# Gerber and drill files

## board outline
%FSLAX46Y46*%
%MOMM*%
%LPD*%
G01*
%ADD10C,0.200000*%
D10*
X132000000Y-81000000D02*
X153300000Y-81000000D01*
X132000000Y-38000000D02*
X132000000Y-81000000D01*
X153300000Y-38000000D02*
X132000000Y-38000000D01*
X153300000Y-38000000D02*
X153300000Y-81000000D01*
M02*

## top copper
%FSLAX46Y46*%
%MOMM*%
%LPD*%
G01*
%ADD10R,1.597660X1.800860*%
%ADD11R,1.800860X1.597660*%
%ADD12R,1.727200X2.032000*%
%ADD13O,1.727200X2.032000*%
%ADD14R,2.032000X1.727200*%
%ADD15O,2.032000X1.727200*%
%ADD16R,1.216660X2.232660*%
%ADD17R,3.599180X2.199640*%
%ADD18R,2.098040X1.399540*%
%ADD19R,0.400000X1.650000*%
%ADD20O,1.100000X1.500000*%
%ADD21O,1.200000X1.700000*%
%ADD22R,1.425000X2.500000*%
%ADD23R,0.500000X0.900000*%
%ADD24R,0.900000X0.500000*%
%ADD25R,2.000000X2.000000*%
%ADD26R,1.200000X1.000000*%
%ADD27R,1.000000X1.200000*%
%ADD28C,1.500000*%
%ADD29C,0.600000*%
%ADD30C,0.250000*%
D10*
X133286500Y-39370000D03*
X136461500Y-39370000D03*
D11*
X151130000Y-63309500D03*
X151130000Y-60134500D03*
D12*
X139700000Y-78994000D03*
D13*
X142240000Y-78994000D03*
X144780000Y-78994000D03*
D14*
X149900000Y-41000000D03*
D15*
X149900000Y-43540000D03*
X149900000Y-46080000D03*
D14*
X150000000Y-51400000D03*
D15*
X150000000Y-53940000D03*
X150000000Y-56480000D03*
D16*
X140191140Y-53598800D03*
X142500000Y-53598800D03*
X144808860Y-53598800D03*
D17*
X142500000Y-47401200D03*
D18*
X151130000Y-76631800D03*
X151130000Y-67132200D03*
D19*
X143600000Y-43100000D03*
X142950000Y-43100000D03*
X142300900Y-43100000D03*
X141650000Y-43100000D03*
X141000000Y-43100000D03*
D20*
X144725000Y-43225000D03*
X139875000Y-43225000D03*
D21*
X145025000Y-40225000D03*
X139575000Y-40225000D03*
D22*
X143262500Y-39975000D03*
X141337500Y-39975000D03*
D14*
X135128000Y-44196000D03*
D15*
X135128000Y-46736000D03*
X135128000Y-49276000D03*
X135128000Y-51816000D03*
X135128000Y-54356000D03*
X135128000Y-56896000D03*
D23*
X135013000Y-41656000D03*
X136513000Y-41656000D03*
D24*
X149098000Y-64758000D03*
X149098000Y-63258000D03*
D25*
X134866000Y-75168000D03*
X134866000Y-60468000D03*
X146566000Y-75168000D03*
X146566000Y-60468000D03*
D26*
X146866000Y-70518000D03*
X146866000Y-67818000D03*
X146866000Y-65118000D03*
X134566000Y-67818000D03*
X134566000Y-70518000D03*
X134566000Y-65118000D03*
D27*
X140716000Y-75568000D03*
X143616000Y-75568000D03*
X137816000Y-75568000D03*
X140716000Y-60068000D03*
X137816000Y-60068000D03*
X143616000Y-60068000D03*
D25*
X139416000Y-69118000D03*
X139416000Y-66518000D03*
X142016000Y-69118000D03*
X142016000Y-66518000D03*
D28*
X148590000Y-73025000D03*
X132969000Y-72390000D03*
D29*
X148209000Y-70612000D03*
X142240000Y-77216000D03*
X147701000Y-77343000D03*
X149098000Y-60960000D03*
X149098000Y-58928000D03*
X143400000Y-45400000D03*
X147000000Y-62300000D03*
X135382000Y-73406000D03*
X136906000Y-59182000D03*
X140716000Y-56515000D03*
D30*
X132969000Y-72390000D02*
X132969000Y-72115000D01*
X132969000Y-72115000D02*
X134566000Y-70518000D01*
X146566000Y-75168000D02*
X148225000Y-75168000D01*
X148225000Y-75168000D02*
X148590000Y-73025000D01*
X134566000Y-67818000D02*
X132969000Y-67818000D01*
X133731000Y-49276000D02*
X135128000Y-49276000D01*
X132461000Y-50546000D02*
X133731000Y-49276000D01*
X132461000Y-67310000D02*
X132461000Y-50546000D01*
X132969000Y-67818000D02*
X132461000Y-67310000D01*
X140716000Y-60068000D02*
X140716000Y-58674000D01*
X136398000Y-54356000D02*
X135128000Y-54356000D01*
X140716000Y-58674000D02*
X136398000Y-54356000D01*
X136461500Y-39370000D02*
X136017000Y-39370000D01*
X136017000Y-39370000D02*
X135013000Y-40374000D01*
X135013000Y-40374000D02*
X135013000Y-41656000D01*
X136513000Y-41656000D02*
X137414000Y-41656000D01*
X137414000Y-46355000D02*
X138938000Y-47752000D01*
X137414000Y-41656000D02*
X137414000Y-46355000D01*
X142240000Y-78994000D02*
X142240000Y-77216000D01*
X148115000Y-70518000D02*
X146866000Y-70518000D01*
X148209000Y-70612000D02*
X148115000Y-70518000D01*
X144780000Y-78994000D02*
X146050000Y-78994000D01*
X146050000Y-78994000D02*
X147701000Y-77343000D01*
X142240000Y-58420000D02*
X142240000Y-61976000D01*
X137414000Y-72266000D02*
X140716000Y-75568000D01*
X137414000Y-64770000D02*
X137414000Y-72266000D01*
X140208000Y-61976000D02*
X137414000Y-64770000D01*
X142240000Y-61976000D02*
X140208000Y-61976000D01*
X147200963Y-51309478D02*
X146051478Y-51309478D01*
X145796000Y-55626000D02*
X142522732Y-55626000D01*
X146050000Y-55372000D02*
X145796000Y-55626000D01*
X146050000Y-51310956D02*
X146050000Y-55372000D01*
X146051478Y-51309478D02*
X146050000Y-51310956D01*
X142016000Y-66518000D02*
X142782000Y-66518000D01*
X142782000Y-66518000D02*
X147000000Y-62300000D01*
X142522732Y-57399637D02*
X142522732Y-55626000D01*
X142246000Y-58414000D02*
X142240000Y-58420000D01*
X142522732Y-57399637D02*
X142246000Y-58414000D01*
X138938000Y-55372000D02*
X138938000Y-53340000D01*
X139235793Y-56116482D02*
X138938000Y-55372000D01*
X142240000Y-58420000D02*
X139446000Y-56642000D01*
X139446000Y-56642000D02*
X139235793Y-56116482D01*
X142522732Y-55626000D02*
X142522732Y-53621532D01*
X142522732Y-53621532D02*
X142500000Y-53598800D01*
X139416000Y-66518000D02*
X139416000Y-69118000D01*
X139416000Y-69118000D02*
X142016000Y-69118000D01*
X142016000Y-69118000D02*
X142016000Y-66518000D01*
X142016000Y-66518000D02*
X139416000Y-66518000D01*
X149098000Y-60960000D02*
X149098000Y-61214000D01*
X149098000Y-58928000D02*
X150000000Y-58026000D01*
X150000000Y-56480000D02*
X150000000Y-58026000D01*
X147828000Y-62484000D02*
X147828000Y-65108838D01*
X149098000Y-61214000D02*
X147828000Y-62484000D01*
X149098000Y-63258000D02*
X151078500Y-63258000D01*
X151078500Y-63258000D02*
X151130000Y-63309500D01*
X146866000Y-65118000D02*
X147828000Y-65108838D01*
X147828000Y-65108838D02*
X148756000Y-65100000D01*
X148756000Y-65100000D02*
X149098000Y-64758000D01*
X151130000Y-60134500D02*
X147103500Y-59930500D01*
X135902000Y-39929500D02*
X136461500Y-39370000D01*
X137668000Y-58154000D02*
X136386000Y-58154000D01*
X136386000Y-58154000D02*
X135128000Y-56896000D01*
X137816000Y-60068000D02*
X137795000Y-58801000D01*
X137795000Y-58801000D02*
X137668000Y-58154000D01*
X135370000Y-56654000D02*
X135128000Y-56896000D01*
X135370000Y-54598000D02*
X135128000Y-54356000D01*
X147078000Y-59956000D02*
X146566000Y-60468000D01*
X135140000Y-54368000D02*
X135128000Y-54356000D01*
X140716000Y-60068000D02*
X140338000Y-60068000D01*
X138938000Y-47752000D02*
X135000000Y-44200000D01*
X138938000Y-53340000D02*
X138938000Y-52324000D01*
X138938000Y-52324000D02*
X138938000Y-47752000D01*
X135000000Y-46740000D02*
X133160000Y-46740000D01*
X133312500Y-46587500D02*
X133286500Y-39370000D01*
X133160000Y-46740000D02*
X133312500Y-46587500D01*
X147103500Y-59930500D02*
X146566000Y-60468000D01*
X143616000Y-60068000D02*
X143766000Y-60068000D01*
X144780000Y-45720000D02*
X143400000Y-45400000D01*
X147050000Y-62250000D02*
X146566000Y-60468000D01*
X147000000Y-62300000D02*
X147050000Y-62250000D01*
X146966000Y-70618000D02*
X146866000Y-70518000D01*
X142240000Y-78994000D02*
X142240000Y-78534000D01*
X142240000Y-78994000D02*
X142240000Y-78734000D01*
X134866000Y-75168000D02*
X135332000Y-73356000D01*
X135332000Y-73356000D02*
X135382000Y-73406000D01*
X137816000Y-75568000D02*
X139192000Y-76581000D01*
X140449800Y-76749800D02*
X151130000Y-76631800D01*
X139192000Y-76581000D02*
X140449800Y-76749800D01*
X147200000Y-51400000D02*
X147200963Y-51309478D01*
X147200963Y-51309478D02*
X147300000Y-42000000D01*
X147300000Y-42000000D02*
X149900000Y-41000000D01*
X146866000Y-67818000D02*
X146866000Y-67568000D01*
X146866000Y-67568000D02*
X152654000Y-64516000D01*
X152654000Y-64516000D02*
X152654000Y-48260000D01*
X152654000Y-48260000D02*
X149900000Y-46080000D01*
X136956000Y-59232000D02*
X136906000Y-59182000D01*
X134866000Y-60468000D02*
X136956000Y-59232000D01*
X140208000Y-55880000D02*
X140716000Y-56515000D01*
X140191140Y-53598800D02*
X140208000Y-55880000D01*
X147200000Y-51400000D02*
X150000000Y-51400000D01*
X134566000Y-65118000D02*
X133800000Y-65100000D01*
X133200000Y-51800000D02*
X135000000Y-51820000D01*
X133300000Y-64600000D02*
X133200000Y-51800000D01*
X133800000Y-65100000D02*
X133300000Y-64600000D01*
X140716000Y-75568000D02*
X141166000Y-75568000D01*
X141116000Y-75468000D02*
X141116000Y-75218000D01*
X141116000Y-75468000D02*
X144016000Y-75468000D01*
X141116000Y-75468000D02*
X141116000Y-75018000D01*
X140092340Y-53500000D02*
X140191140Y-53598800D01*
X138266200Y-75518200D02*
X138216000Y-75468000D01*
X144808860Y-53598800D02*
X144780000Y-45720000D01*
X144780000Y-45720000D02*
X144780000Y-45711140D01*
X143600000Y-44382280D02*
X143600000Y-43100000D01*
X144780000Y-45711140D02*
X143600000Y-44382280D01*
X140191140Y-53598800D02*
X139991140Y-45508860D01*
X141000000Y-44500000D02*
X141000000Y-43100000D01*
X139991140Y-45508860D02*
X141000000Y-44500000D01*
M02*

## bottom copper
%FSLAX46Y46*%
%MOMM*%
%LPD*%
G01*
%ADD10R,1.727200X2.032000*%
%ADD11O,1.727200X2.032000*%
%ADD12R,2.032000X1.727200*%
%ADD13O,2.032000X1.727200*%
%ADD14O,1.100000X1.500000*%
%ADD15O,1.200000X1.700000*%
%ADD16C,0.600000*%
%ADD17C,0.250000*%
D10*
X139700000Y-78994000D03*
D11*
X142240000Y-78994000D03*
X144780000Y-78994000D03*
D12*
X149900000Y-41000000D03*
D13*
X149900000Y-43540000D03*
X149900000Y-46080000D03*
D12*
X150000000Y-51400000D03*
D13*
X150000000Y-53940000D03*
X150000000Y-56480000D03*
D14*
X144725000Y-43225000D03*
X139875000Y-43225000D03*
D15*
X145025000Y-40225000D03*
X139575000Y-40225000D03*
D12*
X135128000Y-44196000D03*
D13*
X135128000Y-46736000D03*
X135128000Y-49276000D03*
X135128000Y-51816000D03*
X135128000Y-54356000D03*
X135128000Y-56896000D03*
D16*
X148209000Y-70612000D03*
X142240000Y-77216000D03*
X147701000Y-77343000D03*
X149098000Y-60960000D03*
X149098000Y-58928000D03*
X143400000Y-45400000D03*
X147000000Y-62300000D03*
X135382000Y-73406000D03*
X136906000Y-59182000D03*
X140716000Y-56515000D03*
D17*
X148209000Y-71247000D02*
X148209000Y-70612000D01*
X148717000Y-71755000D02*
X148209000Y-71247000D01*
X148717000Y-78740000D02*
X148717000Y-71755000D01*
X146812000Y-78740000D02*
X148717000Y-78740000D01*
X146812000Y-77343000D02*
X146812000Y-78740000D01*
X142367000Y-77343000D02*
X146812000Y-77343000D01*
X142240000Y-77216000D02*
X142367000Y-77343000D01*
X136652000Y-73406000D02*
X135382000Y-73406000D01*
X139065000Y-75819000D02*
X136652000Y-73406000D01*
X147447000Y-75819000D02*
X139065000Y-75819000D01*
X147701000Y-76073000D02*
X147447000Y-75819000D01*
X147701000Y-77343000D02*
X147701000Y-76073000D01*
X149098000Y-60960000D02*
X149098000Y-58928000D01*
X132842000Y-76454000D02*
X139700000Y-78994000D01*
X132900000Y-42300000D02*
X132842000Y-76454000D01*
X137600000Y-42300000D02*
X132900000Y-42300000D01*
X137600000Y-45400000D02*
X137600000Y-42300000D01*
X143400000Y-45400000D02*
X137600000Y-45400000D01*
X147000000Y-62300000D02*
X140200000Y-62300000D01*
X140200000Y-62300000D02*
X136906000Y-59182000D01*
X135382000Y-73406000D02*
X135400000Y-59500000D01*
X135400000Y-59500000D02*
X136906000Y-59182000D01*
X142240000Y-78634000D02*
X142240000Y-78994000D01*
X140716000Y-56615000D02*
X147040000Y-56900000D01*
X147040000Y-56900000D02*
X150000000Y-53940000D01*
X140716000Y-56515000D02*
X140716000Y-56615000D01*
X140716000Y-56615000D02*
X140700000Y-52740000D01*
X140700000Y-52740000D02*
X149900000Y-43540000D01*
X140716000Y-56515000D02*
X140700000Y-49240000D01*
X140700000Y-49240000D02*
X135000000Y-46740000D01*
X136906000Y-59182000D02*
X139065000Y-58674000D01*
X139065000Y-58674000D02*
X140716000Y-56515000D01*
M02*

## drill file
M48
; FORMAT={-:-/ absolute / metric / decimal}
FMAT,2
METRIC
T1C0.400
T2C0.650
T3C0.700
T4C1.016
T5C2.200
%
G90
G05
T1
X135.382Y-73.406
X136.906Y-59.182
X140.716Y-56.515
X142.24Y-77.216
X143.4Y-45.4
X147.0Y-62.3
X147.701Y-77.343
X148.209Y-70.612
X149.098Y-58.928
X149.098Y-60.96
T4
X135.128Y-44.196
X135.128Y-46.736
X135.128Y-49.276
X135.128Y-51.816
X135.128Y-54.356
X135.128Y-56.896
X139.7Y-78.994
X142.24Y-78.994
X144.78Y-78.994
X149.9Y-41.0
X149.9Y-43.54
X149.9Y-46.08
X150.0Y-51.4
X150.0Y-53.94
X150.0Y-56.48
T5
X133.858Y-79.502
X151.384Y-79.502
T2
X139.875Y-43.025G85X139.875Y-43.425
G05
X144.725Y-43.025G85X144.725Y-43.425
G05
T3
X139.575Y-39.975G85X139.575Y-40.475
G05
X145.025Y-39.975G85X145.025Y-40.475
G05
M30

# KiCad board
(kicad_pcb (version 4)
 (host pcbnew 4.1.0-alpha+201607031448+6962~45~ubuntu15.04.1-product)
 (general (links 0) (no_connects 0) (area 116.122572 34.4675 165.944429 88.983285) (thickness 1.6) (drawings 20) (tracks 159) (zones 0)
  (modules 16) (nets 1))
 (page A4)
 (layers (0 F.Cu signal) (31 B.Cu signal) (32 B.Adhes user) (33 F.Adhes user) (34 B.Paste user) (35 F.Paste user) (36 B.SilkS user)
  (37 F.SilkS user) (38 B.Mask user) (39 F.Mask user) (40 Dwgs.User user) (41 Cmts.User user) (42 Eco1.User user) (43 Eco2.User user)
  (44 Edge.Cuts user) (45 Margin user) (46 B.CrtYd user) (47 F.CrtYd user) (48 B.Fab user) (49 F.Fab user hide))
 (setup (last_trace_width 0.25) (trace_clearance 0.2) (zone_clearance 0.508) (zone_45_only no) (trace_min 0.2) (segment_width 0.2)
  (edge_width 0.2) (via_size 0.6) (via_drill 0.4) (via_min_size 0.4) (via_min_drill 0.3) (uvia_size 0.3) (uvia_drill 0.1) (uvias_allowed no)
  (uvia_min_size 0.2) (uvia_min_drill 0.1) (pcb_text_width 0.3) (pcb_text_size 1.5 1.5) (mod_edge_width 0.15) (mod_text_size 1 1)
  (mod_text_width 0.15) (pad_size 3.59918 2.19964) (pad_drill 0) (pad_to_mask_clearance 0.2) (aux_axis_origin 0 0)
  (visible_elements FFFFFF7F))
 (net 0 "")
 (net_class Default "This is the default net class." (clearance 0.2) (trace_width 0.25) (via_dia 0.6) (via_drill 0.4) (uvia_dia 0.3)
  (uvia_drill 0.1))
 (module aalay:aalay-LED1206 (layer F.Cu) (at 134.874 39.37)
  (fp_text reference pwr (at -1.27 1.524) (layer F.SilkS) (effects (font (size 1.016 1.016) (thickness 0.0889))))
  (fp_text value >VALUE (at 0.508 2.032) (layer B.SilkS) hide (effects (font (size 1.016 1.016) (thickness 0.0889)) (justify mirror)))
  (pad A smd rect (at -1.5875 0) (size 1.59766 1.80086) (layers F.Cu F.Paste F.Mask))
  (pad K smd rect (at 1.5875 0) (size 1.59766 1.80086) (layers F.Cu F.Paste F.Mask)))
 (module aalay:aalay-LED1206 (layer F.Cu) (at 151.13 61.722 90)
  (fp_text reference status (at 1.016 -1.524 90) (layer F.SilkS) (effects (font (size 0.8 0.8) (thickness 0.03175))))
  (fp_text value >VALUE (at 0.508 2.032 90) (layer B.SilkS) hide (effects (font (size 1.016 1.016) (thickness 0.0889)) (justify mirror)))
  (pad A smd rect (at -1.5875 0 90) (size 1.59766 1.80086) (layers F.Cu F.Paste F.Mask))
  (pad K smd rect (at 1.5875 0 90) (size 1.59766 1.80086) (layers F.Cu F.Paste F.Mask)))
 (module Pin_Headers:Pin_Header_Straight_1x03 (layer F.Cu) (at 139.7 78.994 90)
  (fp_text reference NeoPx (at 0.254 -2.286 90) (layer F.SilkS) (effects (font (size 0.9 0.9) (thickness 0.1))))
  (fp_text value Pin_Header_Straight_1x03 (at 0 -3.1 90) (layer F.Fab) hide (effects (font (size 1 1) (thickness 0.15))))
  (pad 1 thru_hole rect (at 0 0 90) (size 2.032 1.7272) (drill 1.016) (layers *.Cu *.Mask F.SilkS))
  (pad 2 thru_hole oval (at 0 2.54 90) (size 2.032 1.7272) (drill 1.016) (layers *.Cu *.Mask F.SilkS))
  (pad 3 thru_hole oval (at 0 5.08 90) (size 2.032 1.7272) (drill 1.016) (layers *.Cu *.Mask F.SilkS)))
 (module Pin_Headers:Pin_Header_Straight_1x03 (layer F.Cu) (at 149.9 41)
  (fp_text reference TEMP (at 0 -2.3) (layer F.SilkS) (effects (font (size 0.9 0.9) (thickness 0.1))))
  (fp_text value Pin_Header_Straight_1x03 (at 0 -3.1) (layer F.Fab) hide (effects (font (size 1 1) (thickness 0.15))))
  (pad 1 thru_hole rect (at 0 0) (size 2.032 1.7272) (drill 1.016) (layers *.Cu *.Mask F.SilkS))
  (pad 2 thru_hole oval (at 0 2.54) (size 2.032 1.7272) (drill 1.016) (layers *.Cu *.Mask F.SilkS))
  (pad 3 thru_hole oval (at 0 5.08) (size 2.032 1.7272) (drill 1.016) (layers *.Cu *.Mask F.SilkS)))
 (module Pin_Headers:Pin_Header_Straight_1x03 (layer F.Cu) (at 150 51.4)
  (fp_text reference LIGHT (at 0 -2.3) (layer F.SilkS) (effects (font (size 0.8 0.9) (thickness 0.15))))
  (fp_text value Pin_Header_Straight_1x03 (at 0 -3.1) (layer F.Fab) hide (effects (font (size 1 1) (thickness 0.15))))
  (pad 1 thru_hole rect (at 0 0) (size 2.032 1.7272) (drill 1.016) (layers *.Cu *.Mask F.SilkS))
  (pad 2 thru_hole oval (at 0 2.54) (size 2.032 1.7272) (drill 1.016) (layers *.Cu *.Mask F.SilkS))
  (pad 3 thru_hole oval (at 0 5.08) (size 2.032 1.7272) (drill 1.016) (layers *.Cu *.Mask F.SilkS)))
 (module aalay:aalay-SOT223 (layer F.Cu) (at 142.5 50.5)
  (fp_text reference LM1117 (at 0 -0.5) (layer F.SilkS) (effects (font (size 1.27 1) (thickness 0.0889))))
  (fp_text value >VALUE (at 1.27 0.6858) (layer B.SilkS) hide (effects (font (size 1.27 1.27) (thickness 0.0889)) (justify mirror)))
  (pad GND smd rect (at -2.30886 3.0988) (size 1.21666 2.23266) (layers F.Cu F.Paste F.Mask))
  (pad OUT smd rect (at 0 3.0988) (size 1.21666 2.23266) (layers F.Cu F.Paste F.Mask))
  (pad IN smd rect (at 2.30886 3.0988) (size 1.21666 2.23266) (layers F.Cu F.Paste F.Mask))
  (pad OUT smd rect (at 0 -3.0988) (size 3.59918 2.19964) (layers F.Cu F.Paste F.Mask)))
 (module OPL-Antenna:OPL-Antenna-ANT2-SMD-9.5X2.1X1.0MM (layer F.Cu) (at 151.13 71.882 90)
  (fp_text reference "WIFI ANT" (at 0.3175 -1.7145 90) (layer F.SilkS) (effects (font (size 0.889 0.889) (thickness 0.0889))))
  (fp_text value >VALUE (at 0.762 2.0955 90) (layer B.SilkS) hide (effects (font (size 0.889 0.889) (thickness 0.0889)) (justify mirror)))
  (pad 1 smd rect (at -4.7498 0 90) (size 1.39954 2.09804) (layers F.Cu F.Paste F.Mask))
  (pad 2 smd rect (at 4.7498 0 90) (size 1.39954 2.09804) (layers F.Cu F.Paste F.Mask)))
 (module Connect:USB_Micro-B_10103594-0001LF (layer F.Cu) (at 142.3 41.6 180)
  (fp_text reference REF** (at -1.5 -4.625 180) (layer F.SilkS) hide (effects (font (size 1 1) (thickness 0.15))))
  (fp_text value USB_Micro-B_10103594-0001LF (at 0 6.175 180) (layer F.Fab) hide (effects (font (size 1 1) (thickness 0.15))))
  (pad +5 smd rect (at -1.3 -1.5 270) (size 1.65 0.4) (layers F.Cu F.Paste F.Mask))
  (pad D- smd rect (at -0.65 -1.5 270) (size 1.65 0.4) (layers F.Cu F.Paste F.Mask))
  (pad D+ smd rect (at -0.0009 -1.5 270) (size 1.65 0.4) (layers F.Cu F.Paste F.Mask))
  (pad ID smd rect (at 0.65 -1.5 270) (size 1.65 0.4) (layers F.Cu F.Paste F.Mask))
  (pad GND smd rect (at 1.3 -1.5 270) (size 1.65 0.4) (layers F.Cu F.Paste F.Mask))
  (pad 6 thru_hole oval (at -2.425 -1.625 270) (size 1.5 1.1) (drill oval 1.05 0.65) (layers *.Cu *.Mask F.SilkS))
  (pad 6 thru_hole oval (at 2.425 -1.625 270) (size 1.5 1.1) (drill oval 1.05 0.65) (layers *.Cu *.Mask F.SilkS))
  (pad 6 thru_hole oval (at -2.725 1.375 270) (size 1.7 1.2) (drill oval 1.2 0.7) (layers *.Cu *.Mask F.SilkS))
  (pad 6 thru_hole oval (at 2.725 1.375 270) (size 1.7 1.2) (drill oval 1.2 0.7) (layers *.Cu *.Mask F.SilkS))
  (pad 6 smd rect (at -0.9625 1.625 270) (size 2.5 1.425) (layers F.Cu F.Paste F.Mask))
  (pad 6 smd rect (at 0.9625 1.625 270) (size 2.5 1.425) (layers F.Cu F.Paste F.Mask)))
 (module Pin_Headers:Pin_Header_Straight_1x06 (layer F.Cu) (at 135.128 44.196)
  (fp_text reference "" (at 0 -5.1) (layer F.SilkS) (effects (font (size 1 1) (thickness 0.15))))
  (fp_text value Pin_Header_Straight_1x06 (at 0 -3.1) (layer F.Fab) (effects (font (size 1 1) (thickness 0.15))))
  (pad 1 thru_hole rect (at 0 0) (size 2.032 1.7272) (drill 1.016) (layers *.Cu *.Mask F.SilkS))
  (pad 2 thru_hole oval (at 0 2.54) (size 2.032 1.7272) (drill 1.016) (layers *.Cu *.Mask F.SilkS))
  (pad 3 thru_hole oval (at 0 5.08) (size 2.032 1.7272) (drill 1.016) (layers *.Cu *.Mask F.SilkS))
  (pad 4 thru_hole oval (at 0 7.62) (size 2.032 1.7272) (drill 1.016) (layers *.Cu *.Mask F.SilkS))
  (pad 5 thru_hole oval (at 0 10.16) (size 2.032 1.7272) (drill 1.016) (layers *.Cu *.Mask F.SilkS))
  (pad 6 thru_hole oval (at 0 12.7) (size 2.032 1.7272) (drill 1.016) (layers *.Cu *.Mask F.SilkS)))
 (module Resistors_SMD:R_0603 (layer F.Cu) (at 135.763 41.656)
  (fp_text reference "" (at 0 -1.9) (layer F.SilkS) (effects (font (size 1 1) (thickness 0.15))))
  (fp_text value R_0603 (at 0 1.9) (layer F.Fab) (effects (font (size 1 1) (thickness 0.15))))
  (pad 1 smd rect (at -0.75 0) (size 0.5 0.9) (layers F.Cu F.Paste F.Mask))
  (pad 2 smd rect (at 0.75 0) (size 0.5 0.9) (layers F.Cu F.Paste F.Mask)))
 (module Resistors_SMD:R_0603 (layer F.Cu) (at 149.098 64.008 90)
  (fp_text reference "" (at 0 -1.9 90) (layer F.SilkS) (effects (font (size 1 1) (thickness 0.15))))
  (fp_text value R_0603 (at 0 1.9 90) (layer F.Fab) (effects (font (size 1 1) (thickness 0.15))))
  (pad 1 smd rect (at -0.75 0 90) (size 0.5 0.9) (layers F.Cu F.Paste F.Mask))
  (pad 2 smd rect (at 0.75 0 90) (size 0.5 0.9) (layers F.Cu F.Paste F.Mask)))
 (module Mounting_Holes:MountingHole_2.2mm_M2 (layer F.Cu) (at 133.858 79.502)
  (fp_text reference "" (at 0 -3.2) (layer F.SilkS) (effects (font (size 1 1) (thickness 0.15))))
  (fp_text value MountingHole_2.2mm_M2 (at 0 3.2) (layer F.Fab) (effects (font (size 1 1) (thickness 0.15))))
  (pad 1 np_thru_hole circle (at 0 0) (size 2.2 2.2) (drill 2.2) (layers *.Cu *.Mask F.SilkS)))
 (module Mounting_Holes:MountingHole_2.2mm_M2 (layer F.Cu) (at 151.384 79.502)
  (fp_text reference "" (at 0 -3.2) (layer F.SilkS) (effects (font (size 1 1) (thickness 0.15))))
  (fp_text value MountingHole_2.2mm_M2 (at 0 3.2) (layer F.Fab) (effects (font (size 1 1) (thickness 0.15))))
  (pad 1 np_thru_hole circle (at 0 0) (size 2.2 2.2) (drill 2.2) (layers *.Cu *.Mask F.SilkS)))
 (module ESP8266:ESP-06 (layer F.Cu) (at 140.716 67.818 90)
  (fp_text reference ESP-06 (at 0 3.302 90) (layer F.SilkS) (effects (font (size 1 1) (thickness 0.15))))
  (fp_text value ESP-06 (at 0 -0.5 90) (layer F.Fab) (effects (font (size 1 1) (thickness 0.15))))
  (pad GND smd rect (at -7.35 -5.85 90) (size 2 2) (layers F.Cu F.Paste F.Mask))
  (pad GP5 smd rect (at 7.35 -5.85 90) (size 2 2) (layers F.Cu F.Paste F.Mask))
  (pad GP16 smd rect (at -7.35 5.85 90) (size 2 2) (layers F.Cu F.Paste F.Mask))
  (pad GP15 smd rect (at 7.35 5.85 90) (size 2 2) (layers F.Cu F.Paste F.Mask))
  (pad GP14 smd rect (at -2.7 6.15 90) (size 1 1.2) (layers F.Cu F.Paste F.Mask))
  (pad GP12 smd rect (at 0 6.15 90) (size 1 1.2) (layers F.Cu F.Paste F.Mask))
  (pad GP13 smd rect (at 2.7 6.15 90) (size 1 1.2) (layers F.Cu F.Paste F.Mask))
  (pad TX smd rect (at 0 -6.15 90) (size 1 1.2) (layers F.Cu F.Paste F.Mask))
  (pad RST smd rect (at -2.7 -6.15 90) (size 1 1.2) (layers F.Cu F.Paste F.Mask))
  (pad RX smd rect (at 2.7 -6.15 90) (size 1 1.2) (layers F.Cu F.Paste F.Mask))
  (pad 3.3 smd rect (at -7.75 0 90) (size 1.2 1) (layers F.Cu F.Paste F.Mask))
  (pad CHPD smd rect (at -7.75 2.9 90) (size 1.2 1) (layers F.Cu F.Paste F.Mask))
  (pad ANT smd rect (at -7.75 -2.9 90) (size 1.2 1) (layers F.Cu F.Paste F.Mask))
  (pad GP2 smd rect (at 7.75 0 90) (size 1.2 1) (layers F.Cu F.Paste F.Mask))
  (pad GP0 smd rect (at 7.75 -2.9 90) (size 1.2 1) (layers F.Cu F.Paste F.Mask))
  (pad GP4 smd rect (at 7.75 2.9 90) (size 1.2 1) (layers F.Cu F.Paste F.Mask))
  (pad GND smd rect (at -1.3 -1.3 90) (size 2 2) (layers F.Cu F.Paste F.Mask))
  (pad GND smd rect (at 1.3 -1.3 90) (size 2 2) (layers F.Cu F.Paste F.Mask))
  (pad GND smd rect (at -1.3 1.3 90) (size 2 2) (layers F.Cu F.Paste F.Mask))
  (pad GND smd rect (at 1.3 1.3 90) (size 2 2) (layers F.Cu F.Paste F.Mask)))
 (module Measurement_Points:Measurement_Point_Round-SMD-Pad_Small (layer F.Cu) (at 148.59 73.025)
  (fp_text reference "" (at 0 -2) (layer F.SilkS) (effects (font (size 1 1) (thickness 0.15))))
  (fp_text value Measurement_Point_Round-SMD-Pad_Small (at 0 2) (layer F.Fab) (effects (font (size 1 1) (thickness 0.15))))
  (pad 1 smd circle (at 0 0) (size 1.5 1.5) (layers F.Cu F.Mask)))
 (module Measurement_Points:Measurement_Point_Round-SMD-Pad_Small (layer F.Cu) (at 132.969 72.39)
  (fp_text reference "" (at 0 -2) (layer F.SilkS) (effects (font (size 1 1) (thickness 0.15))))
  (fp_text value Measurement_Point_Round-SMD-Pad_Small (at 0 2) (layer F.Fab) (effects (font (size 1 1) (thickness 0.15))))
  (pad 1 smd circle (at 0 0) (size 1.5 1.5) (layers F.Cu F.Mask)))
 (gr_line (start 132 81) (end 153.3 81) (angle 90) (layer Edge.Cuts) (width 0.2))
 (gr_line (start 132 38) (end 132 81) (angle 90) (layer Edge.Cuts) (width 0.2))
 (gr_line (start 153.3 38) (end 132 38) (angle 90) (layer Edge.Cuts) (width 0.2))
 (gr_line (start 153.3 38) (end 153.3 81) (angle 90) (layer Edge.Cuts) (width 0.2))
 (segment (start 132.969 72.39) (end 132.969 72.115) (width 0.25) (layer F.Cu) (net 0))
 (segment (start 132.969 72.115) (end 134.566 70.518) (width 0.25) (layer F.Cu) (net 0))
 (segment (start 146.566 75.168) (end 148.225 75.168) (width 0.25) (layer F.Cu) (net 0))
 (segment (start 148.225 75.168) (end 148.59 73.025) (width 0.25) (layer F.Cu) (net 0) (status 20))
 (segment (start 134.566 67.818) (end 132.969 67.818) (width 0.25) (layer F.Cu) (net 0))
 (segment (start 133.731 49.276) (end 135.128 49.276) (width 0.25) (layer F.Cu) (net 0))
 (segment (start 132.461 50.546) (end 133.731 49.276) (width 0.25) (layer F.Cu) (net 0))
 (segment (start 132.461 67.31) (end 132.461 50.546) (width 0.25) (layer F.Cu) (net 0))
 (segment (start 132.969 67.818) (end 132.461 67.31) (width 0.25) (layer F.Cu) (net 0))
 (segment (start 140.716 60.068) (end 140.716 58.674) (width 0.25) (layer F.Cu) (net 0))
 (segment (start 136.398 54.356) (end 135.128 54.356) (width 0.25) (layer F.Cu) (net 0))
 (segment (start 140.716 58.674) (end 136.398 54.356) (width 0.25) (layer F.Cu) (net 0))
 (segment (start 136.4615 39.37) (end 136.017 39.37) (width 0.25) (layer F.Cu) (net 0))
 (segment (start 136.017 39.37) (end 135.013 40.374) (width 0.25) (layer F.Cu) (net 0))
 (segment (start 135.013 40.374) (end 135.013 41.656) (width 0.25) (layer F.Cu) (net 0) (status 20))
 (segment (start 136.513 41.656) (end 137.414 41.656) (width 0.25) (layer F.Cu) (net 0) (status 10))
 (segment (start 137.414 46.355) (end 138.938 47.752) (width 0.25) (layer F.Cu) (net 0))
 (segment (start 137.414 41.656) (end 137.414 46.355) (width 0.25) (layer F.Cu) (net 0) (status 10))
 (segment (start 142.24 78.994) (end 142.24 77.216) (width 0.25) (layer F.Cu) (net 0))
 (segment (start 148.115 70.518) (end 146.866 70.518) (width 0.25) (layer F.Cu) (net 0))
 (segment (start 148.209 70.612) (end 148.115 70.518) (width 0.25) (layer F.Cu) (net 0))
 (via (at 148.209 70.612) (size 0.6) (drill 0.4) (layers F.Cu B.Cu) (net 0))
 (segment (start 148.209 71.247) (end 148.209 70.612) (width 0.25) (layer B.Cu) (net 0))
 (segment (start 148.717 71.755) (end 148.209 71.247) (width 0.25) (layer B.Cu) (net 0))
 (segment (start 148.717 78.74) (end 148.717 71.755) (width 0.25) (layer B.Cu) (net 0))
 (segment (start 146.812 78.74) (end 148.717 78.74) (width 0.25) (layer B.Cu) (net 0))
 (segment (start 146.812 77.343) (end 146.812 78.74) (width 0.25) (layer B.Cu) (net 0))
 (segment (start 142.367 77.343) (end 146.812 77.343) (width 0.25) (layer B.Cu) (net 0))
 (segment (start 142.24 77.216) (end 142.367 77.343) (width 0.25) (layer B.Cu) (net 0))
 (via (at 142.24 77.216) (size 0.6) (drill 0.4) (layers F.Cu B.Cu) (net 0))
 (segment (start 144.78 78.994) (end 146.05 78.994) (width 0.25) (layer F.Cu) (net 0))
 (segment (start 136.652 73.406) (end 135.382 73.406) (width 0.25) (layer B.Cu) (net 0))
 (segment (start 139.065 75.819) (end 136.652 73.406) (width 0.25) (layer B.Cu) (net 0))
 (segment (start 147.447 75.819) (end 139.065 75.819) (width 0.25) (layer B.Cu) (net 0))
 (segment (start 147.701 76.073) (end 147.447 75.819) (width 0.25) (layer B.Cu) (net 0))
 (segment (start 147.701 77.343) (end 147.701 76.073) (width 0.25) (layer B.Cu) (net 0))
 (via (at 147.701 77.343) (size 0.6) (drill 0.4) (layers F.Cu B.Cu) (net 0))
 (segment (start 146.05 78.994) (end 147.701 77.343) (width 0.25) (layer F.Cu) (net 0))
 (segment (start 142.24 58.42) (end 142.24 61.976) (width 0.25) (layer F.Cu) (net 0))
 (segment (start 137.414 72.266) (end 140.716 75.568) (width 0.25) (layer F.Cu) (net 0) (status 20))
 (segment (start 137.414 64.77) (end 137.414 72.266) (width 0.25) (layer F.Cu) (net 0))
 (segment (start 140.208 61.976) (end 137.414 64.77) (width 0.25) (layer F.Cu) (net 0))
 (segment (start 142.24 61.976) (end 140.208 61.976) (width 0.25) (layer F.Cu) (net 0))
 (segment (start 147.200963 51.309478) (end 146.051478 51.309478) (width 0.25) (layer F.Cu) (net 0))
 (segment (start 145.796 55.626) (end 142.522732 55.626) (width 0.25) (layer F.Cu) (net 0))
 (segment (start 146.05 55.372) (end 145.796 55.626) (width 0.25) (layer F.Cu) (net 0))
 (segment (start 146.05 51.310956) (end 146.05 55.372) (width 0.25) (layer F.Cu) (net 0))
 (segment (start 146.051478 51.309478) (end 146.05 51.310956) (width 0.25) (layer F.Cu) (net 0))
 (segment (start 142.016 66.518) (end 142.782 66.518) (width 0.25) (layer F.Cu) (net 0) (status 30))
 (segment (start 142.782 66.518) (end 147 62.3) (width 0.25) (layer F.Cu) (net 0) (status 10))
 (segment (start 142.522732 57.399637) (end 142.522732 55.626) (width 0.25) (layer F.Cu) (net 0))
 (segment (start 142.246 58.414) (end 142.24 58.42) (width 0.25) (layer F.Cu) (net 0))
 (segment (start 142.522732 57.399637) (end 142.246 58.414) (width 0.25) (layer F.Cu) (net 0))
 (segment (start 138.938 55.372) (end 138.938 53.34) (width 0.25) (layer F.Cu) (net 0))
 (segment (start 139.235793 56.116482) (end 138.938 55.372) (width 0.25) (layer F.Cu) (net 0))
 (segment (start 142.24 58.42) (end 139.446 56.642) (width 0.25) (layer F.Cu) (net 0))
 (segment (start 139.446 56.642) (end 139.235793 56.116482) (width 0.25) (layer F.Cu) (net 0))
 (segment (start 142.522732 55.626) (end 142.522732 53.621532) (width 0.25) (layer F.Cu) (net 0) (status 20))
 (segment (start 142.522732 53.621532) (end 142.5 53.5988) (width 0.25) (layer F.Cu) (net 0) (status 30))
 (segment (start 139.416 66.518) (end 139.416 69.118) (width 0.25) (layer F.Cu) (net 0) (status 30))
 (segment (start 139.416 69.118) (end 142.016 69.118) (width 0.25) (layer F.Cu) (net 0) (status 30))
 (segment (start 142.016 69.118) (end 142.016 66.518) (width 0.25) (layer F.Cu) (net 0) (status 30))
 (segment (start 142.016 66.518) (end 139.416 66.518) (width 0.25) (layer F.Cu) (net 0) (status 30))
 (segment (start 149.098 60.96) (end 149.098 61.214) (width 0.25) (layer F.Cu) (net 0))
 (via (at 149.098 60.96) (size 0.6) (drill 0.4) (layers F.Cu B.Cu) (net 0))
 (segment (start 149.098 60.96) (end 149.098 58.928) (width 0.25) (layer B.Cu) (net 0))
 (via (at 149.098 58.928) (size 0.6) (drill 0.4) (layers F.Cu B.Cu) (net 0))
 (segment (start 149.098 58.928) (end 150 58.026) (width 0.25) (layer F.Cu) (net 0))
 (segment (start 150 56.48) (end 150 58.026) (width 0.25) (layer F.Cu) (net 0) (status 10))
 (segment (start 147.828 62.484) (end 147.828 65.108838) (width 0.25) (layer F.Cu) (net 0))
 (segment (start 149.098 61.214) (end 147.828 62.484) (width 0.25) (layer F.Cu) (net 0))
 (segment (start 149.098 63.258) (end 151.0785 63.258) (width 0.25) (layer F.Cu) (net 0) (status 30))
 (segment (start 151.0785 63.258) (end 151.13 63.3095) (width 0.25) (layer F.Cu) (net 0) (status 30))
 (segment (start 146.866 65.118) (end 147.828 65.108838) (width 0.25) (layer F.Cu) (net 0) (status 10))
 (segment (start 147.828 65.108838) (end 148.756 65.1) (width 0.25) (layer F.Cu) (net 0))
 (segment (start 148.756 65.1) (end 149.098 64.758) (width 0.25) (layer F.Cu) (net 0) (status 20))
 (segment (start 151.13 60.1345) (end 147.1035 59.9305) (width 0.25) (layer F.Cu) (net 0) (status 30))
 (segment (start 135.902 39.9295) (end 136.4615 39.37) (width 0.25) (layer F.Cu) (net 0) (status 30))
 (segment (start 137.668 58.154) (end 136.386 58.154) (width 0.25) (layer F.Cu) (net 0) (status 10))
 (segment (start 136.386 58.154) (end 135.128 56.896) (width 0.25) (layer F.Cu) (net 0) (status 20))
 (segment (start 137.816 60.068) (end 137.795 58.801) (width 0.25) (layer F.Cu) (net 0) (status 10))
 (segment (start 137.795 58.801) (end 137.668 58.154) (width 0.25) (layer F.Cu) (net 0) (status 20))
 (segment (start 135.37 56.654) (end 135.128 56.896) (width 0.25) (layer F.Cu) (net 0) (status 30))
 (segment (start 135.37 54.598) (end 135.128 54.356) (width 0.25) (layer F.Cu) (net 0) (status 30))
 (segment (start 147.078 59.956) (end 146.566 60.468) (width 0.25) (layer F.Cu) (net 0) (status 30))
 (segment (start 135.14 54.368) (end 135.128 54.356) (width 0.25) (layer F.Cu) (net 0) (status 30))
 (segment (start 140.716 60.068) (end 140.338 60.068) (width 0.25) (layer F.Cu) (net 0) (status 30))
 (segment (start 138.938 47.752) (end 135 44.2) (width 0.25) (layer F.Cu) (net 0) (status 20))
 (segment (start 138.938 53.34) (end 138.938 52.324) (width 0.25) (layer F.Cu) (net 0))
 (segment (start 138.938 52.324) (end 138.938 47.752) (width 0.25) (layer F.Cu) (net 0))
 (segment (start 135 46.74) (end 133.16 46.74) (width 0.25) (layer F.Cu) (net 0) (status 10))
 (segment (start 133.3125 46.5875) (end 133.2865 39.37) (width 0.25) (layer F.Cu) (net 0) (status 20))
 (segment (start 133.16 46.74) (end 133.3125 46.5875) (width 0.25) (layer F.Cu) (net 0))
 (segment (start 147.1035 59.9305) (end 146.566 60.468) (width 0.25) (layer F.Cu) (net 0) (status 30))
 (segment (start 143.616 60.068) (end 143.766 60.068) (width 0.25) (layer F.Cu) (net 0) (status 30))
 (segment (start 144.78 45.72) (end 143.4 45.4) (width 0.25) (layer F.Cu) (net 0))
 (segment (start 132.842 76.454) (end 139.7 78.994) (width 0.25) (layer B.Cu) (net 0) (status 20))
 (segment (start 132.9 42.3) (end 132.842 76.454) (width 0.25) (layer B.Cu) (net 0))
 (segment (start 137.6 42.3) (end 132.9 42.3) (width 0.25) (layer B.Cu) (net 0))
 (segment (start 137.6 45.4) (end 137.6 42.3) (width 0.25) (layer B.Cu) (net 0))
 (segment (start 143.4 45.4) (end 137.6 45.4) (width 0.25) (layer B.Cu) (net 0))
 (via (at 143.4 45.4) (size 0.6) (drill 0.4) (layers F.Cu B.Cu) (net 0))
 (segment (start 147 62.3) (end 140.2 62.3) (width 0.25) (layer B.Cu) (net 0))
 (segment (start 140.2 62.3) (end 136.906 59.182) (width 0.25) (layer B.Cu) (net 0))
 (segment (start 147.05 62.25) (end 146.566 60.468) (width 0.25) (layer F.Cu) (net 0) (status 20))
 (via (at 147 62.3) (size 0.6) (drill 0.4) (layers F.Cu B.Cu) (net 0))
 (segment (start 147 62.3) (end 147.05 62.25) (width 0.25) (layer F.Cu) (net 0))
 (segment (start 146.966 70.618) (end 146.866 70.518) (width 0.25) (layer F.Cu) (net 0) (status 30))
 (segment (start 142.24 78.994) (end 142.24 78.534) (width 0.25) (layer F.Cu) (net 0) (status 30))
 (segment (start 142.24 78.994) (end 142.24 78.734) (width 0.25) (layer F.Cu) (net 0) (status 30))
 (segment (start 135.382 73.406) (end 135.4 59.5) (width 0.25) (layer B.Cu) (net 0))
 (via (at 135.382 73.406) (size 0.6) (drill 0.4) (layers F.Cu B.Cu) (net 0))
 (segment (start 134.866 75.168) (end 135.332 73.356) (width 0.25) (layer F.Cu) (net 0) (status 10))
 (segment (start 135.332 73.356) (end 135.382 73.406) (width 0.25) (layer F.Cu) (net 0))
 (segment (start 135.4 59.5) (end 136.906 59.182) (width 0.25) (layer B.Cu) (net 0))
 (segment (start 142.24 78.634) (end 142.24 78.994) (width 0.25) (layer B.Cu) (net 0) (status 30))
 (segment (start 137.816 75.568) (end 139.192 76.581) (width 0.25) (layer F.Cu) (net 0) (status 10))
 (segment (start 140.4498 76.7498) (end 151.13 76.6318) (width 0.25) (layer F.Cu) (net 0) (status 20))
 (segment (start 139.192 76.581) (end 140.4498 76.7498) (width 0.25) (layer F.Cu) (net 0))
 (segment (start 147.2 51.4) (end 147.200963 51.309478) (width 0.25) (layer F.Cu) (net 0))
 (segment (start 147.200963 51.309478) (end 147.3 42) (width 0.25) (layer F.Cu) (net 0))
 (segment (start 147.3 42) (end 149.9 41) (width 0.25) (layer F.Cu) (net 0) (status 20))
 (segment (start 140.716 56.615) (end 147.04 56.9) (width 0.25) (layer B.Cu) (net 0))
 (segment (start 147.04 56.9) (end 150 53.94) (width 0.25) (layer B.Cu) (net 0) (status 20))
 (segment (start 146.866 67.818) (end 146.866 67.568) (width 0.25) (layer F.Cu) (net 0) (status 30))
 (segment (start 146.866 67.568) (end 152.654 64.516) (width 0.25) (layer F.Cu) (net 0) (status 10))
 (segment (start 152.654 64.516) (end 152.654 48.26) (width 0.25) (layer F.Cu) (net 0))
 (segment (start 152.654 48.26) (end 149.9 46.08) (width 0.25) (layer F.Cu) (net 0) (status 20))
 (segment (start 140.716 56.515) (end 140.716 56.615) (width 0.25) (layer B.Cu) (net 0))
 (segment (start 140.716 56.615) (end 140.7 52.74) (width 0.25) (layer B.Cu) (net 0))
 (segment (start 140.7 52.74) (end 149.9 43.54) (width 0.25) (layer B.Cu) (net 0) (status 20))
 (segment (start 140.716 56.515) (end 140.7 49.24) (width 0.25) (layer B.Cu) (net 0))
 (segment (start 140.7 49.24) (end 135 46.74) (width 0.25) (layer B.Cu) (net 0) (status 20))
 (segment (start 136.906 59.182) (end 139.065 58.674) (width 0.25) (layer B.Cu) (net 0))
 (segment (start 139.065 58.674) (end 140.716 56.515) (width 0.25) (layer B.Cu) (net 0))
 (segment (start 136.956 59.232) (end 136.906 59.182) (width 0.25) (layer F.Cu) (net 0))
 (via (at 136.906 59.182) (size 0.6) (drill 0.4) (layers F.Cu B.Cu) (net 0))
 (segment (start 134.866 60.468) (end 136.956 59.232) (width 0.25) (layer F.Cu) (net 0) (status 10))
 (segment (start 140.208 55.88) (end 140.716 56.515) (width 0.25) (layer F.Cu) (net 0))
 (via (at 140.716 56.515) (size 0.6) (drill 0.4) (layers F.Cu B.Cu) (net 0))
 (segment (start 140.19114 53.5988) (end 140.208 55.88) (width 0.25) (layer F.Cu) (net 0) (status 10))
 (segment (start 147.2 51.4) (end 150 51.4) (width 0.25) (layer F.Cu) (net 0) (status 20))
 (segment (start 134.566 65.118) (end 133.8 65.1) (width 0.25) (layer F.Cu) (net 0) (status 10))
 (segment (start 133.2 51.8) (end 135 51.82) (width 0.25) (layer F.Cu) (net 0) (status 20))
 (segment (start 133.3 64.6) (end 133.2 51.8) (width 0.25) (layer F.Cu) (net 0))
 (segment (start 133.8 65.1) (end 133.3 64.6) (width 0.25) (layer F.Cu) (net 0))
 (segment (start 140.716 75.568) (end 141.166 75.568) (width 0.25) (layer F.Cu) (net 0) (status 30))
 (segment (start 141.116 75.468) (end 141.116 75.218) (width 0.25) (layer F.Cu) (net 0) (status 30))
 (segment (start 141.116 75.468) (end 144.016 75.468) (width 0.25) (layer F.Cu) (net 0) (status 30))
 (segment (start 141.116 75.468) (end 141.116 75.018) (width 0.25) (layer F.Cu) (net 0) (status 30))
 (segment (start 140.09234 53.5) (end 140.19114 53.5988) (width 0.25) (layer F.Cu) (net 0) (status 30))
 (segment (start 138.2662 75.5182) (end 138.216 75.468) (width 0.25) (layer F.Cu) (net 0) (status 30))
 (segment (start 144.80886 53.5988) (end 144.78 45.72) (width 0.25) (layer F.Cu) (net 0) (status 10))
 (segment (start 144.78 45.72) (end 144.78 45.71114) (width 0.25) (layer F.Cu) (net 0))
 (segment (start 143.6 44.38228) (end 143.6 43.1) (width 0.25) (layer F.Cu) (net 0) (status 20))
 (segment (start 144.78 45.71114) (end 143.6 44.38228) (width 0.25) (layer F.Cu) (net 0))
 (segment (start 140.19114 53.5988) (end 139.99114 45.50886) (width 0.25) (layer F.Cu) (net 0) (status 10))
 (segment (start 141 44.5) (end 141 43.1) (width 0.25) (layer F.Cu) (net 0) (status 20))
 (segment (start 139.99114 45.50886) (end 141 44.5) (width 0.25) (layer F.Cu) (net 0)))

